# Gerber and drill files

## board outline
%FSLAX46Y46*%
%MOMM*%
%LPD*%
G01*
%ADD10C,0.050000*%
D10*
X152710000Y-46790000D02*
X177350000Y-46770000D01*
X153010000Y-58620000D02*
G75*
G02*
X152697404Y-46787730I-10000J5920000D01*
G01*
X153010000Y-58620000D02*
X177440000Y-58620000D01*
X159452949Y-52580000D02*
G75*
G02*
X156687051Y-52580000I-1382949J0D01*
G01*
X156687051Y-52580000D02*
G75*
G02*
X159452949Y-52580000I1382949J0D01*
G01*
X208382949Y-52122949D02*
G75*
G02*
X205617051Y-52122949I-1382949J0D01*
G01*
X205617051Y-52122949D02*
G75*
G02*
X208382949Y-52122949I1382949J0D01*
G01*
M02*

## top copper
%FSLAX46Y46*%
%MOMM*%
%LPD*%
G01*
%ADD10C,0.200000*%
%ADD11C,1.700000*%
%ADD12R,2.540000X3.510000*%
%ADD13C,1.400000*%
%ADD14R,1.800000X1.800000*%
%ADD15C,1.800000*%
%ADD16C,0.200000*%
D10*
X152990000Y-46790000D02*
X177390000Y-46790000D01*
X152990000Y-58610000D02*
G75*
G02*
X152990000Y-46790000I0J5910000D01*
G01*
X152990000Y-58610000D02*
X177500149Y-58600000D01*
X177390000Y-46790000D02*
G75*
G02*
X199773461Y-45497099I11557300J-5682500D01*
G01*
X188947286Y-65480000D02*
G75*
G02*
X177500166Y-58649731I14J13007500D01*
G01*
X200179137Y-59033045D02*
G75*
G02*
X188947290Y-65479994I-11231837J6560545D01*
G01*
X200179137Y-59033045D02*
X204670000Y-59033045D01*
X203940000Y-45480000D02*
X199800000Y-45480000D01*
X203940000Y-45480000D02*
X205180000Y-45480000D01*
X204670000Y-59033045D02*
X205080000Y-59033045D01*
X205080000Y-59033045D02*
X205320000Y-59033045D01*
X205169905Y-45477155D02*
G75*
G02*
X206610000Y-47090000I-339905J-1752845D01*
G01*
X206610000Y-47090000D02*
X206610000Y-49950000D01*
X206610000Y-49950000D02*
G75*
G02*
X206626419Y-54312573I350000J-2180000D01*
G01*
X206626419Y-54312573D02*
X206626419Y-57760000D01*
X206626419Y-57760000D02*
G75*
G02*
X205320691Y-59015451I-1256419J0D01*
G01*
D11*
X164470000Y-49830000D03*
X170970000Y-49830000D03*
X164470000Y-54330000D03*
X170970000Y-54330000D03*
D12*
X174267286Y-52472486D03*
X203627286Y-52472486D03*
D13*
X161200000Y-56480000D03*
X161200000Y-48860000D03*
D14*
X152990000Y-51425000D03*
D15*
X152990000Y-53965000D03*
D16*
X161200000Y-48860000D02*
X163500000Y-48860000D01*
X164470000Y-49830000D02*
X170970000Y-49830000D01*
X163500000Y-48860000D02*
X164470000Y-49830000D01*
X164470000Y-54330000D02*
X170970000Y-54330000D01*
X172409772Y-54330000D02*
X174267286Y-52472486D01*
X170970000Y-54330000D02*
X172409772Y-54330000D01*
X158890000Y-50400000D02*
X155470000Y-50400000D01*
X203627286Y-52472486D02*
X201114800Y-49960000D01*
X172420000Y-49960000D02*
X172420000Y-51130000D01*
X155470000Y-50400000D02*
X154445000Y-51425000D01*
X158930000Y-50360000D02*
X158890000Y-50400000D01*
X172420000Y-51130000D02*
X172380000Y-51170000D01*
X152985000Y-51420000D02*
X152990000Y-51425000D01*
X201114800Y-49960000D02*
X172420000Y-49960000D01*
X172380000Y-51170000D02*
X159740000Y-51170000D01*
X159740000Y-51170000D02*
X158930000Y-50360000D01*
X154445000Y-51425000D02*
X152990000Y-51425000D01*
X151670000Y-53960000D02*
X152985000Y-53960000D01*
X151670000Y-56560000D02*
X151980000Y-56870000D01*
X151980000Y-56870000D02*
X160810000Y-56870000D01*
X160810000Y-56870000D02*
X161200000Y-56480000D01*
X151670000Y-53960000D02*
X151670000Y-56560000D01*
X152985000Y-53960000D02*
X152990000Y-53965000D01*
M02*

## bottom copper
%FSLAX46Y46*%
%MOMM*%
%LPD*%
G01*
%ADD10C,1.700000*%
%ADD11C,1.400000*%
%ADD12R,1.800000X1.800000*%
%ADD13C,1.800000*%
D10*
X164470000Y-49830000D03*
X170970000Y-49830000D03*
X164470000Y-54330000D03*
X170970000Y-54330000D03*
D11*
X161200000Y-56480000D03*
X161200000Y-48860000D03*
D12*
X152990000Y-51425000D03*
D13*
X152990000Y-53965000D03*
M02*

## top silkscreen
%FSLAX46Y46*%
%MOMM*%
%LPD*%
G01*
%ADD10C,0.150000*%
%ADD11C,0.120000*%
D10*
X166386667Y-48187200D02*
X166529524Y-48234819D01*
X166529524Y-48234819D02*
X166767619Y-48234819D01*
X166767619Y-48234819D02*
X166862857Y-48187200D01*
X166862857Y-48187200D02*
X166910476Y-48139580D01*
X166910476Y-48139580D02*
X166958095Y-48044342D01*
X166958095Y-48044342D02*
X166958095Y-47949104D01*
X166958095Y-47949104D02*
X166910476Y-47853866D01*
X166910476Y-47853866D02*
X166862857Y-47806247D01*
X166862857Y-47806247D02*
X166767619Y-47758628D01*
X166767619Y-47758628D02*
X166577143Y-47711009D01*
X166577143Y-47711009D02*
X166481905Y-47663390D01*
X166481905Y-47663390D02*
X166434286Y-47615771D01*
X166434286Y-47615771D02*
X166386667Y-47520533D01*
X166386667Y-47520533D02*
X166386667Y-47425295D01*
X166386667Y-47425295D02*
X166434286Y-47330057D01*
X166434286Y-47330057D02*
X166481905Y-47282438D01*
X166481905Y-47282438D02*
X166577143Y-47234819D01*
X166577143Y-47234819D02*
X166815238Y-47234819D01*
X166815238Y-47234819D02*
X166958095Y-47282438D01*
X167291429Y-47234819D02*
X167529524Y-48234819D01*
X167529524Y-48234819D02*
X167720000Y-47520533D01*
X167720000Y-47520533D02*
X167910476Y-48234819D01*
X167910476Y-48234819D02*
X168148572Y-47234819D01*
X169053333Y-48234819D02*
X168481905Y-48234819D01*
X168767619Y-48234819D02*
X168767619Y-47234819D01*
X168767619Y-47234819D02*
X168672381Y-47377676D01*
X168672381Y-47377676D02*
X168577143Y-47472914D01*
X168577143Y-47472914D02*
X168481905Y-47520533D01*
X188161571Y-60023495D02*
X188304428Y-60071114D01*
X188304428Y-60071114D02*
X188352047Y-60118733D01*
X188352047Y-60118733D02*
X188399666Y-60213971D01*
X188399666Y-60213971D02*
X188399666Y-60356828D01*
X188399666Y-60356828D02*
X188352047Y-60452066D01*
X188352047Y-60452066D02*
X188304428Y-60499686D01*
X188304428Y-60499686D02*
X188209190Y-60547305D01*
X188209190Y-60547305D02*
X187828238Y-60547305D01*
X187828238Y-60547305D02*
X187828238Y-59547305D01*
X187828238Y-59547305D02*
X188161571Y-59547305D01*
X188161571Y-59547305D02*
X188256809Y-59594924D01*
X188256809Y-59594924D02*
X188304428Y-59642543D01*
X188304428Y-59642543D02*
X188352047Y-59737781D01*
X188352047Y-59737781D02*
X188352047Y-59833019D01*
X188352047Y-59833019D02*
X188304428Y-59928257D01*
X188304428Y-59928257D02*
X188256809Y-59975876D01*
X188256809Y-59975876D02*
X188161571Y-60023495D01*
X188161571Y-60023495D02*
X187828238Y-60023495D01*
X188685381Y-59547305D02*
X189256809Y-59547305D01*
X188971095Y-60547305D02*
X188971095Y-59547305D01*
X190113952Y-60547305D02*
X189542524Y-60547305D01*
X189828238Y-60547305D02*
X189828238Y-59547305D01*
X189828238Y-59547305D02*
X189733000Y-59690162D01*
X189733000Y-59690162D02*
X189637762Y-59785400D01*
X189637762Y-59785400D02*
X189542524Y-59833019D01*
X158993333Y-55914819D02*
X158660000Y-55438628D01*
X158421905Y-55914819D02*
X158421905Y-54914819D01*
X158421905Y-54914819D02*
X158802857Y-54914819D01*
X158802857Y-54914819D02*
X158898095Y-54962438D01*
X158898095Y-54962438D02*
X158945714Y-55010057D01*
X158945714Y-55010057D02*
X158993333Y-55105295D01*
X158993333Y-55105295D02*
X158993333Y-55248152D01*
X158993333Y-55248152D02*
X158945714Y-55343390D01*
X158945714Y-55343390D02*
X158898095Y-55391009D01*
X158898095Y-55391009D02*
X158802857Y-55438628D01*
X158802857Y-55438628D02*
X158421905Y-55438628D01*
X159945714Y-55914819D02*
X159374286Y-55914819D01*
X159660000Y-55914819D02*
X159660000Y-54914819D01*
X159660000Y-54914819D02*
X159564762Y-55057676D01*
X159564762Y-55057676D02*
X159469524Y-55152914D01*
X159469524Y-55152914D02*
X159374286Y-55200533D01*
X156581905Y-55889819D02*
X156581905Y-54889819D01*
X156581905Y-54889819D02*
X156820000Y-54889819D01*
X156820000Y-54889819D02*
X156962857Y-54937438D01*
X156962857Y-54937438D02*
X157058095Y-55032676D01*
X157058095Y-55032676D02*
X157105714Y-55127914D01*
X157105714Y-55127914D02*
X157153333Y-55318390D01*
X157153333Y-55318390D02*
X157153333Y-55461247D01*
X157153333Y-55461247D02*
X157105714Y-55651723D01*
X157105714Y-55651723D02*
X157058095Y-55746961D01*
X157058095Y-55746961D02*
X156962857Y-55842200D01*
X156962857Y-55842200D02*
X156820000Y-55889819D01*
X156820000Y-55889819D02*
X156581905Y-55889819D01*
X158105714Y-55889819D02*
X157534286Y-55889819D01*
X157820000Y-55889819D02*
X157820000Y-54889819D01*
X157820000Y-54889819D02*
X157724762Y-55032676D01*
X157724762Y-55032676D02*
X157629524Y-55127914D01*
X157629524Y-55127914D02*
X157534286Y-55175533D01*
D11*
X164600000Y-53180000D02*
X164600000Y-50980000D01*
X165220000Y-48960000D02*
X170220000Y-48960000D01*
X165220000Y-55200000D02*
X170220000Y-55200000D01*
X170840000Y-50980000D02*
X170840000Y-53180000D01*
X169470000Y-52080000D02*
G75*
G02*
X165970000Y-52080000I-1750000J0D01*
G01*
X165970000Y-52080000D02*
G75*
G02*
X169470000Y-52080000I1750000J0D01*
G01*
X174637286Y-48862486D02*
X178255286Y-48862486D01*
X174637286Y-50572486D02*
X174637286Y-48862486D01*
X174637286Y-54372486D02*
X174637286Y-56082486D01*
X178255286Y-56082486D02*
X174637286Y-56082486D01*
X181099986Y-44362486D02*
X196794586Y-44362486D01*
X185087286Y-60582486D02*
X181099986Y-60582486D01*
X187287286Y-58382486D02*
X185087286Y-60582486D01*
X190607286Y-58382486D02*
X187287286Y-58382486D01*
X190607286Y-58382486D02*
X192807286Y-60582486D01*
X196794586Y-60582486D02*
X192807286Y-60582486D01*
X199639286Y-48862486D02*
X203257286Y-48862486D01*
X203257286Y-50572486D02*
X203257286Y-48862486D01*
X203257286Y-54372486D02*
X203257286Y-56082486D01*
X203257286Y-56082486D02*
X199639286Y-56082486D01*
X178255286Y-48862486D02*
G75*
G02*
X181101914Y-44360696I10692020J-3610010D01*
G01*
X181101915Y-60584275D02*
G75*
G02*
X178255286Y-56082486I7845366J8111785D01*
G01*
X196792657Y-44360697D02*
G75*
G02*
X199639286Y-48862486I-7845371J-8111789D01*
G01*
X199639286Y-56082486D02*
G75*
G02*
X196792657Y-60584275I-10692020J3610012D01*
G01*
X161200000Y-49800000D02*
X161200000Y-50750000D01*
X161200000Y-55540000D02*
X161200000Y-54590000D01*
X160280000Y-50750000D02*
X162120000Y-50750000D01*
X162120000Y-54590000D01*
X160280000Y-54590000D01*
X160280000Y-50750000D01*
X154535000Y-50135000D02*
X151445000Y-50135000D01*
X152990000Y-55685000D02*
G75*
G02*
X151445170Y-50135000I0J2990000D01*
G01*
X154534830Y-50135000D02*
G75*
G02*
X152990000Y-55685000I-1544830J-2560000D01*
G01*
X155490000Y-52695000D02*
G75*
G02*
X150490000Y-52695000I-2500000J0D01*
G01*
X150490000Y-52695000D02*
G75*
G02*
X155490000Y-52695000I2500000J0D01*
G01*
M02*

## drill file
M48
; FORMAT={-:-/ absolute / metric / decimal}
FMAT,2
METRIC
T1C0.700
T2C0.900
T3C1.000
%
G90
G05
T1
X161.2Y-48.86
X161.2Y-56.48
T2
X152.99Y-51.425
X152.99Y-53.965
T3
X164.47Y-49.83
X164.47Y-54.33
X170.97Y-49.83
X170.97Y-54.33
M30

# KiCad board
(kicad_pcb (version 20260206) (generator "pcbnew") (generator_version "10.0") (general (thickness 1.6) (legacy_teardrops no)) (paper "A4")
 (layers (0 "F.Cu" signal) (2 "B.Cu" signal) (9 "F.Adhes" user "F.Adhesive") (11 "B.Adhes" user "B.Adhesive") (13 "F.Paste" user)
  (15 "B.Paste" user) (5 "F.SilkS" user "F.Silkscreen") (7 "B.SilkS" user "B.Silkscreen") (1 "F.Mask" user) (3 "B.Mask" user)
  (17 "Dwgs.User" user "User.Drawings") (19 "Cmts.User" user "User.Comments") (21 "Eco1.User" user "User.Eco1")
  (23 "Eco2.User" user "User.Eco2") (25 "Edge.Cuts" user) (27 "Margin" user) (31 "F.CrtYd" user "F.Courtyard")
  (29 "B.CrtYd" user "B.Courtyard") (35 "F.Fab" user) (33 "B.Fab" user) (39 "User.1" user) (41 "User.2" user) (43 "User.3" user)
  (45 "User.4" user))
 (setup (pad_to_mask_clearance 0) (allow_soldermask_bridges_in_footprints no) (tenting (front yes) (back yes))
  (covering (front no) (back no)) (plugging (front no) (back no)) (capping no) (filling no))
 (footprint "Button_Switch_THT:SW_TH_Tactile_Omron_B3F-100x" (layer "F.Cu") (at 164.47 49.83)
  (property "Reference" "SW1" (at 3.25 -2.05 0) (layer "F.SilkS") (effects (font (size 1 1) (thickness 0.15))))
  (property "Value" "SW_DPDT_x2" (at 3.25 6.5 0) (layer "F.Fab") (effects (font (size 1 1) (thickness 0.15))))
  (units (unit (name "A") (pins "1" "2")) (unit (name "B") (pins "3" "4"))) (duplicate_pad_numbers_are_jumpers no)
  (fp_line (start 0.13 3.35) (end 0.13 1.15) (stroke (width 0.12) (type solid)) (layer "F.SilkS"))
  (fp_line (start 0.75 -0.87) (end 5.75 -0.87) (stroke (width 0.12) (type solid)) (layer "F.SilkS"))
  (fp_line (start 0.75 5.37) (end 5.75 5.37) (stroke (width 0.12) (type solid)) (layer "F.SilkS"))
  (fp_line (start 6.37 1.15) (end 6.37 3.35) (stroke (width 0.12) (type solid)) (layer "F.SilkS"))
  (fp_circle (center 3.25 2.25) (end 5 2.25) (stroke (width 0.12) (type solid)) (fill no) (layer "F.SilkS"))
  (pad "1" thru_hole circle (at 0 0) (size 1.7 1.7) (drill 1) (layers "*.Cu" "*.Mask") (remove_unused_layers no) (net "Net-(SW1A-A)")
   (thermal_bridge_angle 90))
  (pad "1" thru_hole circle (at 6.5 0) (size 1.7 1.7) (drill 1) (layers "*.Cu" "*.Mask") (remove_unused_layers no) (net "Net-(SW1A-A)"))
  (pad "2" thru_hole circle (at 0 4.5) (size 1.7 1.7) (drill 1) (layers "*.Cu" "*.Mask") (remove_unused_layers no) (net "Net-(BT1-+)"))
  (pad "2" thru_hole circle (at 6.5 4.5) (size 1.7 1.7) (drill 1) (layers "*.Cu" "*.Mask") (remove_unused_layers no) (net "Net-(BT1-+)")))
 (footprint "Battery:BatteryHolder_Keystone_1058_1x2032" (layer "F.Cu") (at 188.947286 52.472486)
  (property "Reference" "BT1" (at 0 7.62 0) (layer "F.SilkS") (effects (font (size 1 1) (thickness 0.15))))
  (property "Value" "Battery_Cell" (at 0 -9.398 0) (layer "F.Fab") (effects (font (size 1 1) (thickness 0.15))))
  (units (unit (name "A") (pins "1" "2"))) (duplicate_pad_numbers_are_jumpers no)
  (fp_line (start -14.31 -3.61) (end -10.692 -3.61) (stroke (width 0.12) (type solid)) (layer "F.SilkS"))
  (fp_line (start -14.31 -1.9) (end -14.31 -3.61) (stroke (width 0.12) (type solid)) (layer "F.SilkS"))
  (fp_line (start -14.31 1.9) (end -14.31 3.61) (stroke (width 0.12) (type solid)) (layer "F.SilkS"))
  (fp_line (start -10.692 3.61) (end -14.31 3.61) (stroke (width 0.12) (type solid)) (layer "F.SilkS"))
  (fp_line (start -7.8473 -8.11) (end 7.8473 -8.11) (stroke (width 0.12) (type solid)) (layer "F.SilkS"))
  (fp_line (start -3.86 8.11) (end -7.8473 8.11) (stroke (width 0.12) (type solid)) (layer "F.SilkS"))
  (fp_line (start -1.66 5.91) (end -3.86 8.11) (stroke (width 0.12) (type solid)) (layer "F.SilkS"))
  (fp_line (start 1.66 5.91) (end -1.66 5.91) (stroke (width 0.12) (type solid)) (layer "F.SilkS"))
  (fp_line (start 1.66 5.91) (end 3.86 8.11) (stroke (width 0.12) (type solid)) (layer "F.SilkS"))
  (fp_line (start 7.8473 8.11) (end 3.86 8.11) (stroke (width 0.12) (type solid)) (layer "F.SilkS"))
  (fp_line (start 10.692 -3.61) (end 14.31 -3.61) (stroke (width 0.12) (type solid)) (layer "F.SilkS"))
  (fp_line (start 14.31 -1.9) (end 14.31 -3.61) (stroke (width 0.12) (type solid)) (layer "F.SilkS"))
  (fp_line (start 14.31 1.9) (end 14.31 3.61) (stroke (width 0.12) (type solid)) (layer "F.SilkS"))
  (fp_line (start 14.31 3.61) (end 10.692 3.61) (stroke (width 0.12) (type solid)) (layer "F.SilkS"))
  (fp_arc (start -10.692 -3.61) (mid -9.538084 -6.031244) (end -7.845371 -8.111789) (stroke (width 0.12) (type solid)) (layer "F.SilkS"))
  (fp_arc (start -7.845371 8.111789) (mid -9.538085 6.031244) (end -10.692 3.61) (stroke (width 0.12) (type solid)) (layer "F.SilkS"))
  (fp_arc (start 7.845371 -8.111789) (mid 9.538085 -6.031244) (end 10.692 -3.61) (stroke (width 0.12) (type solid)) (layer "F.SilkS"))
  (fp_arc (start 10.692 3.61) (mid 9.538084 6.031244) (end 7.845371 8.111789) (stroke (width 0.12) (type solid)) (layer "F.SilkS"))
  (pad "1" smd rect (at -14.68 0) (size 2.54 3.51) (layers "F.Cu" "F.Mask" "F.Paste") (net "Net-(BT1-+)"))
  (pad "2" smd rect (at 14.68 0) (size 2.54 3.51) (layers "F.Cu" "F.Mask" "F.Paste") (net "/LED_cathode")))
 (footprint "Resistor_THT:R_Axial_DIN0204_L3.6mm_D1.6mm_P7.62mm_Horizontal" (layer "F.Cu") (at 161.2 56.48 90)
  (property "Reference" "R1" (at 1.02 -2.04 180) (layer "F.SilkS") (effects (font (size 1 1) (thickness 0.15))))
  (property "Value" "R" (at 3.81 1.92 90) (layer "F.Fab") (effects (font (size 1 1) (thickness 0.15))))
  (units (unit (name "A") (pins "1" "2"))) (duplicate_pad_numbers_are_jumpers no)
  (fp_line (start 6.68 0) (end 5.73 0) (stroke (width 0.12) (type solid)) (layer "F.SilkS"))
  (fp_line (start 0.94 0) (end 1.89 0) (stroke (width 0.12) (type solid)) (layer "F.SilkS"))
  (fp_rect (start 1.89 -0.92) (end 5.73 0.92) (stroke (width 0.12) (type solid)) (fill no) (layer "F.SilkS"))
  (pad "1" thru_hole circle (at 0 0 90) (size 1.4 1.4) (drill 0.7) (layers "*.Cu" "*.Mask") (remove_unused_layers no) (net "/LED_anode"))
  (pad "2" thru_hole circle (at 7.62 0 90) (size 1.4 1.4) (drill 0.7) (layers "*.Cu" "*.Mask") (remove_unused_layers no)
   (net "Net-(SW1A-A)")))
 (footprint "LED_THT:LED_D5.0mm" (layer "F.Cu") (at 152.99 51.425 -90)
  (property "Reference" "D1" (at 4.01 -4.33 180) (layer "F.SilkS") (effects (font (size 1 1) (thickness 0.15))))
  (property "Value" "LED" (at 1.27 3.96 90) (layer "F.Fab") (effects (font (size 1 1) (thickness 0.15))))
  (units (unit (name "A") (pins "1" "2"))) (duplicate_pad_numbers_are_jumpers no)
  (fp_line (start -1.29 -1.545) (end -1.29 1.545) (stroke (width 0.12) (type solid)) (layer "F.SilkS"))
  (fp_arc (start 4.26 0) (mid 2.071779 2.880495) (end -1.29 1.54483) (stroke (width 0.12) (type solid)) (layer "F.SilkS"))
  (fp_arc (start -1.29 -1.54483) (mid 2.071779 -2.880495) (end 4.26 0) (stroke (width 0.12) (type solid)) (layer "F.SilkS"))
  (fp_circle (center 1.27 0) (end 3.77 0) (stroke (width 0.12) (type solid)) (fill no) (layer "F.SilkS"))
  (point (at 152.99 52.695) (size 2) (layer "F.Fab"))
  (pad "1" thru_hole rect (at 0 0 270) (size 1.8 1.8) (drill 0.9) (layers "*.Cu" "*.Mask") (remove_unused_layers no) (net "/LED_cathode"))
  (pad "2" thru_hole circle (at 2.54 0 270) (size 1.8 1.8) (drill 0.9) (layers "*.Cu" "*.Mask") (remove_unused_layers no) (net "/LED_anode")))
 (gr_line (start 152.99 46.79) (end 177.39 46.79) (stroke (width 0.2) (type default)) (layer "F.Cu"))
 (gr_arc (start 152.99 58.61) (mid 147.08 52.7) (end 152.99 46.79) (stroke (width 0.2) (type default)) (layer "F.Cu"))
 (gr_line (start 152.99 58.61) (end 177.500149 58.6) (stroke (width 0.2) (type default)) (layer "F.Cu"))
 (gr_arc (start 177.39 46.79) (mid 188.204637 39.615193) (end 199.773442 45.497111) (stroke (width 0.2) (type default)) (layer "F.Cu"))
 (gr_arc (start 188.947286 65.48) (mid 182.282277 63.642673) (end 177.500149 58.64974) (stroke (width 0.2) (type default)) (layer "F.Cu"))
 (gr_arc (start 200.179137 59.033045) (mid 195.422581 63.753708) (end 188.94729 65.48) (stroke (width 0.2) (type default)) (layer "F.Cu"))
 (gr_line (start 200.179137 59.033045) (end 204.67 59.033045) (stroke (width 0.2) (type default)) (layer "F.Cu"))
 (gr_line (start 203.94 45.48) (end 199.8 45.48) (stroke (width 0.2) (type default)) (layer "F.Cu"))
 (gr_line (start 203.94 45.48) (end 205.18 45.48) (stroke (width 0.2) (type default)) (layer "F.Cu"))
 (gr_line (start 204.67 59.033045) (end 205.08 59.033045) (stroke (width 0.2) (type default)) (layer "F.Cu"))
 (gr_line (start 205.08 59.033045) (end 205.32 59.033045) (stroke (width 0.2) (type default)) (layer "F.Cu"))
 (gr_arc (start 205.169905 45.477155) (mid 206.161847 46.040805) (end 206.61 47.09) (stroke (width 0.2) (type default)) (layer "F.Cu"))
 (gr_line (start 206.61 47.09) (end 206.61 49.95) (stroke (width 0.2) (type default)) (layer "F.Cu"))
 (gr_arc (start 206.61 49.95) (mid 209.167902 52.12169) (end 206.626419 54.312573) (stroke (width 0.2) (type default)) (layer "F.Cu"))
 (gr_line (start 206.626419 54.312573) (end 206.626419 57.76) (stroke (width 0.2) (type default)) (layer "F.Cu"))
 (gr_arc (start 206.626419 57.76) (mid 206.240815 58.665688) (end 205.320691 59.015451) (stroke (width 0.2) (type default)) (layer "F.Cu"))
 (gr_line (start 152.71 46.79) (end 177.35 46.77) (stroke (width 0.05) (type default)) (layer "Edge.Cuts"))
 (gr_arc (start 153.01 58.62) (mid 147.082056 52.856346) (end 152.697404 46.787731) (stroke (width 0.05) (type default)) (layer "Edge.Cuts"))
 (gr_line (start 153.01 58.62) (end 177.44 58.62) (stroke (width 0.05) (type default)) (layer "Edge.Cuts"))
 (gr_circle (center 158.07 52.58) (end 157.400338 53.79) (stroke (width 0.05) (type default)) (fill no) (layer "Edge.Cuts"))
 (gr_circle (center 207 52.122949) (end 206.330338 53.332949) (stroke (width 0.05) (type default)) (fill no) (layer "Edge.Cuts"))
 (segment (start 161.2 48.86) (end 163.5 48.86) (width 0.2) (layer "F.Cu") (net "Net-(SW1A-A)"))
 (segment (start 164.47 49.83) (end 170.97 49.83) (width 0.2) (layer "F.Cu") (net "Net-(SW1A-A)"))
 (segment (start 163.5 48.86) (end 164.47 49.83) (width 0.2) (layer "F.Cu") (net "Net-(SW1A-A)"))
 (segment (start 164.47 54.33) (end 170.97 54.33) (width 0.2) (layer "F.Cu") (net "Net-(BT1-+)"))
 (segment (start 172.409772 54.33) (end 174.267286 52.472486) (width 0.2) (layer "F.Cu") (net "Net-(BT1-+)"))
 (segment (start 170.97 54.33) (end 172.409772 54.33) (width 0.2) (layer "F.Cu") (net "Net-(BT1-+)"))
 (segment (start 158.89 50.4) (end 155.47 50.4) (width 0.2) (layer "F.Cu") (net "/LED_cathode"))
 (segment (start 203.627286 52.472486) (end 201.1148 49.96) (width 0.2) (layer "F.Cu") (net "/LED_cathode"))
 (segment (start 172.42 49.96) (end 172.42 51.13) (width 0.2) (layer "F.Cu") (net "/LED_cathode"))
 (segment (start 155.47 50.4) (end 154.445 51.425) (width 0.2) (layer "F.Cu") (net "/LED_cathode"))
 (segment (start 158.93 50.36) (end 158.89 50.4) (width 0.2) (layer "F.Cu") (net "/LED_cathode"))
 (segment (start 172.42 51.13) (end 172.38 51.17) (width 0.2) (layer "F.Cu") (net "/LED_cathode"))
 (segment (start 152.985 51.42) (end 152.99 51.425) (width 0.2) (layer "F.Cu") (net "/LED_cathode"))
 (segment (start 201.1148 49.96) (end 172.42 49.96) (width 0.2) (layer "F.Cu") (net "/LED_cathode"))
 (segment (start 172.38 51.17) (end 159.74 51.17) (width 0.2) (layer "F.Cu") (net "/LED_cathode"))
 (segment (start 159.74 51.17) (end 158.93 50.36) (width 0.2) (layer "F.Cu") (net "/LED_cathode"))
 (segment (start 154.445 51.425) (end 152.99 51.425) (width 0.2) (layer "F.Cu") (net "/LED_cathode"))
 (segment (start 151.67 53.96) (end 152.985 53.96) (width 0.2) (layer "F.Cu") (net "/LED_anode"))
 (segment (start 151.67 56.56) (end 151.98 56.87) (width 0.2) (layer "F.Cu") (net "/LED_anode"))
 (segment (start 151.98 56.87) (end 160.81 56.87) (width 0.2) (layer "F.Cu") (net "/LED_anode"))
 (segment (start 160.81 56.87) (end 161.2 56.48) (width 0.2) (layer "F.Cu") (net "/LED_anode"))
 (segment (start 151.67 53.96) (end 151.67 56.56) (width 0.2) (layer "F.Cu") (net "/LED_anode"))
 (segment (start 152.985 53.96) (end 152.99 53.965) (width 0.2) (layer "F.Cu") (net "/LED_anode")))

